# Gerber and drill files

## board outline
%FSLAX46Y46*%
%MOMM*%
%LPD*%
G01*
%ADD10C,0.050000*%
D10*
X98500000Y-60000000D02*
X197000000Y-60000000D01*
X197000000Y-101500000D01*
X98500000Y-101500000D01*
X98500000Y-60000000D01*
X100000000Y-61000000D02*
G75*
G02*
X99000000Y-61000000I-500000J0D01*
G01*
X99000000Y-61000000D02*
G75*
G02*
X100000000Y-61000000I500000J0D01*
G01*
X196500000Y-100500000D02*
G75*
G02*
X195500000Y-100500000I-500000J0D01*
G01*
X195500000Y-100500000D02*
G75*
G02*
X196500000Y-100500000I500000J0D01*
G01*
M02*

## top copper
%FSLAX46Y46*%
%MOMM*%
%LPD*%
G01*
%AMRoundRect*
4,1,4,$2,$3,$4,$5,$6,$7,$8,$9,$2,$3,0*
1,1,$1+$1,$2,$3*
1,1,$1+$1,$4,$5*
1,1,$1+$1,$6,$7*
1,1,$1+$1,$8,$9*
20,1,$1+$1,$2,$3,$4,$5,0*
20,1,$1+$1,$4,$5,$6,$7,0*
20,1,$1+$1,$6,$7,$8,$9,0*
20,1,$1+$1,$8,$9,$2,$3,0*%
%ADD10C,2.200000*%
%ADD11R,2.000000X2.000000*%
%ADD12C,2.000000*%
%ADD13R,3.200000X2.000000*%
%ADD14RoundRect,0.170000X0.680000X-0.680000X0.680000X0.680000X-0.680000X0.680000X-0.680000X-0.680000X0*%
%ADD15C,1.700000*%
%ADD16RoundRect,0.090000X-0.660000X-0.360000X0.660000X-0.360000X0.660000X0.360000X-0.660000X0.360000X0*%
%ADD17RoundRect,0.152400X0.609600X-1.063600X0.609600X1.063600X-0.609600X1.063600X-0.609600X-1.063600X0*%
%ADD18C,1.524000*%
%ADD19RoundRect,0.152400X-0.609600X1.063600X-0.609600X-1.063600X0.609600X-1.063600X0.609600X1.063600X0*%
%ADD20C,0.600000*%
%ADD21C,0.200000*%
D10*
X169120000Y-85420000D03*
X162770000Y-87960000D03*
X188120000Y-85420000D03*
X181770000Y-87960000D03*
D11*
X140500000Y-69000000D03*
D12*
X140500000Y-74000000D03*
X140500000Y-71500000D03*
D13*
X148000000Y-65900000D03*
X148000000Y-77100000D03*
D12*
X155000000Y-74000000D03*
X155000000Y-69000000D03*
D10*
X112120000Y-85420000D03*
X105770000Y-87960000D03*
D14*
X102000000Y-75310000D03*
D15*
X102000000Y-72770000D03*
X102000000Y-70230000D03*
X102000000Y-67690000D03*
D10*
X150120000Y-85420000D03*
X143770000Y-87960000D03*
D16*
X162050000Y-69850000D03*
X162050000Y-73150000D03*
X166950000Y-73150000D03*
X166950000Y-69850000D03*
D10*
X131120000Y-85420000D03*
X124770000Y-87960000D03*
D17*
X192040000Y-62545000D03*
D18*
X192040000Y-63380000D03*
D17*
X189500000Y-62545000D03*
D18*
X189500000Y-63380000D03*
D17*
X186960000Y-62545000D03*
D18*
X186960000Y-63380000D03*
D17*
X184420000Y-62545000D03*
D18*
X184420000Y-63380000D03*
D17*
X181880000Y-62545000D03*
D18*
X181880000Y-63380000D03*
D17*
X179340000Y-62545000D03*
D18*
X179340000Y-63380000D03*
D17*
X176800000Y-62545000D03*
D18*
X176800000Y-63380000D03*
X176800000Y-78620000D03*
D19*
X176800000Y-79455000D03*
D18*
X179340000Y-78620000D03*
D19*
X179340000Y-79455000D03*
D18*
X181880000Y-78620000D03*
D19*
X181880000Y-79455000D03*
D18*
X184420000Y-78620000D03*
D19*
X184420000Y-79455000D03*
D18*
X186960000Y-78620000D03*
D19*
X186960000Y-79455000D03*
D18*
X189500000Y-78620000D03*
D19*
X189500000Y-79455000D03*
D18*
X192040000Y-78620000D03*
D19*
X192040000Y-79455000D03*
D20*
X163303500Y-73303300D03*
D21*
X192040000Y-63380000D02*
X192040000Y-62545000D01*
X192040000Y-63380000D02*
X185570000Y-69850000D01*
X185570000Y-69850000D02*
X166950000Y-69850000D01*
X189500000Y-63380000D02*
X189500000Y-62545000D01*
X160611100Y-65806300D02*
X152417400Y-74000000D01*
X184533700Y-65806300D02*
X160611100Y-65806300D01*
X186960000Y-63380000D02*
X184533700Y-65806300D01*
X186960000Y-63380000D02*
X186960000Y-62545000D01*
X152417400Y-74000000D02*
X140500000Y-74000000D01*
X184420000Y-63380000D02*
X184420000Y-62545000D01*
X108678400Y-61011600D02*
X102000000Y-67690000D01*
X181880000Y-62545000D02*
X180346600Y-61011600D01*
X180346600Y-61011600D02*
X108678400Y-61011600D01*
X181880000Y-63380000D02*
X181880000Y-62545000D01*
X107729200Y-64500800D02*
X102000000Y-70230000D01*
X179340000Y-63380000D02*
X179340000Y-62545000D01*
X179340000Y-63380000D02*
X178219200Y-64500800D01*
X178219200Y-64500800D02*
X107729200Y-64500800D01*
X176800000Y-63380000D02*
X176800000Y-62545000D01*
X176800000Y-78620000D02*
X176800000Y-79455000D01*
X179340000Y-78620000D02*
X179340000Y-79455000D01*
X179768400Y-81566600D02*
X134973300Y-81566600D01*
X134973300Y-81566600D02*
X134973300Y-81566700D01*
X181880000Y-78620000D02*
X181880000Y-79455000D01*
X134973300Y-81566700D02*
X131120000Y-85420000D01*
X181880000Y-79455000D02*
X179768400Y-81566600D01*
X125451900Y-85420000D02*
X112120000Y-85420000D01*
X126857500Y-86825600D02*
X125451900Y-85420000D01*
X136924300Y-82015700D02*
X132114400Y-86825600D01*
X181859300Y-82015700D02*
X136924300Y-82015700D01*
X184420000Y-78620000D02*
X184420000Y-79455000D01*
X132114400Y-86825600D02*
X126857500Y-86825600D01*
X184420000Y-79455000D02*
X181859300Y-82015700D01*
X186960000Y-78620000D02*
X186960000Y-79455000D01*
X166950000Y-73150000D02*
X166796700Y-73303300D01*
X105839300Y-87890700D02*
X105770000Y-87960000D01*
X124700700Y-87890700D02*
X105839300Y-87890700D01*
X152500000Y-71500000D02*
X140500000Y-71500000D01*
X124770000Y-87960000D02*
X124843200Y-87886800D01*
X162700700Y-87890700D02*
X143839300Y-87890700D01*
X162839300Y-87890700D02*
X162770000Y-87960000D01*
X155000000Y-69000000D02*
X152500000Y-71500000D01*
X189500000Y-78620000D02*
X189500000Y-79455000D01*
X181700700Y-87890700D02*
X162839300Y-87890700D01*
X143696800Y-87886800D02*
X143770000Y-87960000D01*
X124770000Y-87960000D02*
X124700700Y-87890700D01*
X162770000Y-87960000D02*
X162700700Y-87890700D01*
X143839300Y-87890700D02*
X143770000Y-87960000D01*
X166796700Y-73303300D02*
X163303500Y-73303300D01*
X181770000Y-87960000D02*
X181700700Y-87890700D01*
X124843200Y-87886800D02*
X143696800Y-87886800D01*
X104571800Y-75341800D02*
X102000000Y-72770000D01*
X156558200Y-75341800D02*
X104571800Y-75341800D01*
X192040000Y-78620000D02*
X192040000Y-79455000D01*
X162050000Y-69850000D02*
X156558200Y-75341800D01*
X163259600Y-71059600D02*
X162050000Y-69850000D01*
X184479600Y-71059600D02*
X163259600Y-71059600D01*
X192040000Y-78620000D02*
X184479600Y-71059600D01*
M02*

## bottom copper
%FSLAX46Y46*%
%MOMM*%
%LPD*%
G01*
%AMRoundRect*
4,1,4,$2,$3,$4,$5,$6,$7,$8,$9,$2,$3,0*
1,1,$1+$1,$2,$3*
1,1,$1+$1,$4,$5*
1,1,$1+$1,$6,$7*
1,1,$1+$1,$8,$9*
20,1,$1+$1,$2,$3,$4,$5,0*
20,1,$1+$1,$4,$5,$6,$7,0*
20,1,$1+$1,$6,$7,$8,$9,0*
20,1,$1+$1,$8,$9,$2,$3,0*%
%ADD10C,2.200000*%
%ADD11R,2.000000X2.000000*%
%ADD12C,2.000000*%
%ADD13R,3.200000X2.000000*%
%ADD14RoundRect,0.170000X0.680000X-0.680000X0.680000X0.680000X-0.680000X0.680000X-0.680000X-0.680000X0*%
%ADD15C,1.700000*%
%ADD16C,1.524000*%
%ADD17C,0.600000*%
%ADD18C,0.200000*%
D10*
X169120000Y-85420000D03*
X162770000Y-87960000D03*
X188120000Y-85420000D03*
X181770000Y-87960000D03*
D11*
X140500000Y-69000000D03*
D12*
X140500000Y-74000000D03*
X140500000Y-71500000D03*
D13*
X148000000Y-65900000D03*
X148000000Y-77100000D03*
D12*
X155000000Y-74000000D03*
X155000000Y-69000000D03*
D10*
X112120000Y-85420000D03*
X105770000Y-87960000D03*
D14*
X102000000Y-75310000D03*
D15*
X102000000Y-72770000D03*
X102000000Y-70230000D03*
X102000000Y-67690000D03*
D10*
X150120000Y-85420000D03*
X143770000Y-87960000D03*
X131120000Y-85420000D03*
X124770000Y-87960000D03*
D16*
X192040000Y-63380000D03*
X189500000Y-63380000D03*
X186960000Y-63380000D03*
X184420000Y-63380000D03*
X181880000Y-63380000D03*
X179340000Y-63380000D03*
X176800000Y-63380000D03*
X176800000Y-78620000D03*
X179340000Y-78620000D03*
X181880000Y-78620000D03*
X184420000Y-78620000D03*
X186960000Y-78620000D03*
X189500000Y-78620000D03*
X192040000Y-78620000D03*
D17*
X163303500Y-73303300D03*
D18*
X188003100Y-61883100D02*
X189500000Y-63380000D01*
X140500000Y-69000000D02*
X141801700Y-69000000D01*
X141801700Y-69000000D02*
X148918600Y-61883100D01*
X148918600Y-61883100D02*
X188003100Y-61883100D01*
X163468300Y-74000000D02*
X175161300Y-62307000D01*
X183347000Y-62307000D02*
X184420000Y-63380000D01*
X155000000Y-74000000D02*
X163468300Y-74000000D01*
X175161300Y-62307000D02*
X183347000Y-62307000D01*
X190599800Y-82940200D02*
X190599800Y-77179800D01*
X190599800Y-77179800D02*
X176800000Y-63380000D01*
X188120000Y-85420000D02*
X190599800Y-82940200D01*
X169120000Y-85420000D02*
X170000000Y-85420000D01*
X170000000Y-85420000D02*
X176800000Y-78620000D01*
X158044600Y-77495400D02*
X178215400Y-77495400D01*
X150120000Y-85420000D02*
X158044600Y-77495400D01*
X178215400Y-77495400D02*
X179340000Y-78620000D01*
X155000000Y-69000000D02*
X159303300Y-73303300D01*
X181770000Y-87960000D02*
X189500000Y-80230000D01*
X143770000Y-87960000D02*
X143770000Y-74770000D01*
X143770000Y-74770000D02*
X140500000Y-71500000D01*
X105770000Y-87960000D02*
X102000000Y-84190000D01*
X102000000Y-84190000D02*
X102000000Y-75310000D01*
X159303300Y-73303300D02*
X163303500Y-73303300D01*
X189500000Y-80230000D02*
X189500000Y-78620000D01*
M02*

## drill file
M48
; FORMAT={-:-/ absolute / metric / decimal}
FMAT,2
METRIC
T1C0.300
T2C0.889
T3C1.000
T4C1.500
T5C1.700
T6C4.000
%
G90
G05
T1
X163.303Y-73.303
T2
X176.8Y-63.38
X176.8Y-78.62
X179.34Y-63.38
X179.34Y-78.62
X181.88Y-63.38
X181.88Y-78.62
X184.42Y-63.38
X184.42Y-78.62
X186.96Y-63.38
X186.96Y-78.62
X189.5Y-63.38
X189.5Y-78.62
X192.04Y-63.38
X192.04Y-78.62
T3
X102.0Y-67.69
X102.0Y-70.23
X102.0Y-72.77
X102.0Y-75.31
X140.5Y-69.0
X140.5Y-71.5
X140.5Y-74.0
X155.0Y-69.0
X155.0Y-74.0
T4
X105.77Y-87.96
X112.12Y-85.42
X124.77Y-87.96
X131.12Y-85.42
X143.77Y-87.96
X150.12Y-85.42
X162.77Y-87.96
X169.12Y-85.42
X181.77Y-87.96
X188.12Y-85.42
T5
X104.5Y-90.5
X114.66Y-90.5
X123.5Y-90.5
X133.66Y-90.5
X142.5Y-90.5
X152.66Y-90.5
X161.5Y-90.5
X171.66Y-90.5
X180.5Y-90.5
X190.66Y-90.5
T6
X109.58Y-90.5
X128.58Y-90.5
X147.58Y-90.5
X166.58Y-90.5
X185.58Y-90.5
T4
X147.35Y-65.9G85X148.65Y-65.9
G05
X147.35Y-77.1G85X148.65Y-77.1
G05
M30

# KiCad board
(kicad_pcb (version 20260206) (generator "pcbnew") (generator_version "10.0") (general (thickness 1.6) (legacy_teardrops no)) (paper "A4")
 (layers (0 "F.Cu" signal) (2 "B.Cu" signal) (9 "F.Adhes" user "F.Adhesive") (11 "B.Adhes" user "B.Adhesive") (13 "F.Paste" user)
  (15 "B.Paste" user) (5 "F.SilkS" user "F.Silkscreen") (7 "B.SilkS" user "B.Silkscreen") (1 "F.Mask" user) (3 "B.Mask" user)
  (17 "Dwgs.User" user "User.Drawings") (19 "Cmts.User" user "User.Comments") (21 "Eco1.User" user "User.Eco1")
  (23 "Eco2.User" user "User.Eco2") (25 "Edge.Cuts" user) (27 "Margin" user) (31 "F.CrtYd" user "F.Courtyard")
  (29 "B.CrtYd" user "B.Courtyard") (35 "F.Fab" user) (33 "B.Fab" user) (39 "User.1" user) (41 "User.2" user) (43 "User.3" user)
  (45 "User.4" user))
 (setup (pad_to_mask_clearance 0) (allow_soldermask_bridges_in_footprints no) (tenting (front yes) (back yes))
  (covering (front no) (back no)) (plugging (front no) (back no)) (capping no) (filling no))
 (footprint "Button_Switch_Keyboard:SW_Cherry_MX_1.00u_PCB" (layer "F.Cu") (at 169.12 85.42)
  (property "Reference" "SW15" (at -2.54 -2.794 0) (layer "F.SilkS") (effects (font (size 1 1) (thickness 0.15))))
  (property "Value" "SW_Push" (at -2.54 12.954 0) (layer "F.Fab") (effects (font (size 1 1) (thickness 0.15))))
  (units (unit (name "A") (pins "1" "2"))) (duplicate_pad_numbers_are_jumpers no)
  (pad "" np_thru_hole circle (at -7.62 5.08) (size 1.7 1.7) (drill 1.7) (layers "*.Cu" "*.Mask"))
  (pad "" np_thru_hole circle (at -2.54 5.08) (size 4 4) (drill 4) (layers "*.Cu" "*.Mask"))
  (pad "" np_thru_hole circle (at 2.54 5.08) (size 1.7 1.7) (drill 1.7) (layers "*.Cu" "*.Mask"))
  (pad "1" thru_hole circle (at 0 0) (size 2.2 2.2) (drill 1.5) (layers "*.Cu" "*.Mask") (remove_unused_layers no)
   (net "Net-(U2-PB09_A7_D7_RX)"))
  (pad "2" thru_hole circle (at -6.35 2.54) (size 2.2 2.2) (drill 1.5) (layers "*.Cu" "*.Mask") (remove_unused_layers no)
   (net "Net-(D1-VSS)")))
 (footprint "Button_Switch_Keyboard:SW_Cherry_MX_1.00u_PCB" (layer "F.Cu") (at 188.12 85.42)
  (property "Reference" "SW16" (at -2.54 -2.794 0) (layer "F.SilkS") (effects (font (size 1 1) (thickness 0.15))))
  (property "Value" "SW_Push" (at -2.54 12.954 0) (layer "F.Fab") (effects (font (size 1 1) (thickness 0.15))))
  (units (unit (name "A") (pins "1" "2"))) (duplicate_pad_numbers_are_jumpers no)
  (pad "" np_thru_hole circle (at -7.62 5.08) (size 1.7 1.7) (drill 1.7) (layers "*.Cu" "*.Mask"))
  (pad "" np_thru_hole circle (at -2.54 5.08) (size 4 4) (drill 4) (layers "*.Cu" "*.Mask"))
  (pad "" np_thru_hole circle (at 2.54 5.08) (size 1.7 1.7) (drill 1.7) (layers "*.Cu" "*.Mask"))
  (pad "1" thru_hole circle (at 0 0) (size 2.2 2.2) (drill 1.5) (layers "*.Cu" "*.Mask") (remove_unused_layers no)
   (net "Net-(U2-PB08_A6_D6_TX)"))
  (pad "2" thru_hole circle (at -6.35 2.54) (size 2.2 2.2) (drill 1.5) (layers "*.Cu" "*.Mask") (remove_unused_layers no)
   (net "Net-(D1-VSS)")))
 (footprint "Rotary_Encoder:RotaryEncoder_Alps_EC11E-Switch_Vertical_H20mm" (layer "F.Cu") (at 140.5 69)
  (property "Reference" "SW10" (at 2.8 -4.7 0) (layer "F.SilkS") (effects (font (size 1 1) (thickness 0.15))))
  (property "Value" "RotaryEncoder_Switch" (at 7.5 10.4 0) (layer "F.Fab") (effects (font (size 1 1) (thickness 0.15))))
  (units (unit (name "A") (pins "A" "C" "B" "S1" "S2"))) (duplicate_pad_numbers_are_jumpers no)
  (pad "A" thru_hole rect (at 0 0) (size 2 2) (drill 1) (layers "*.Cu" "*.Mask") (remove_unused_layers no) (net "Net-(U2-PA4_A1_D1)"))
  (pad "B" thru_hole circle (at 0 5) (size 2 2) (drill 1) (layers "*.Cu" "*.Mask") (remove_unused_layers no) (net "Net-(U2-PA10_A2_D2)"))
  (pad "C" thru_hole circle (at 0 2.5) (size 2 2) (drill 1) (layers "*.Cu" "*.Mask") (remove_unused_layers no) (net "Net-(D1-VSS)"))
  (pad "MP" thru_hole rect (at 7.5 -3.1) (size 3.2 2) (drill oval 2.8 1.5) (layers "*.Cu" "*.Mask") (remove_unused_layers no))
  (pad "MP" thru_hole rect (at 7.5 8.1) (size 3.2 2) (drill oval 2.8 1.5) (layers "*.Cu" "*.Mask") (remove_unused_layers no))
  (pad "S1" thru_hole circle (at 14.5 5) (size 2 2) (drill 1) (layers "*.Cu" "*.Mask") (remove_unused_layers no) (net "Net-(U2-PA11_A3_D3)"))
  (pad "S2" thru_hole circle (at 14.5 0) (size 2 2) (drill 1) (layers "*.Cu" "*.Mask") (remove_unused_layers no) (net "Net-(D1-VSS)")))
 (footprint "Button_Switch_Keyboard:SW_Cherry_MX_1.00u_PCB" (layer "F.Cu") (at 112.12 85.42)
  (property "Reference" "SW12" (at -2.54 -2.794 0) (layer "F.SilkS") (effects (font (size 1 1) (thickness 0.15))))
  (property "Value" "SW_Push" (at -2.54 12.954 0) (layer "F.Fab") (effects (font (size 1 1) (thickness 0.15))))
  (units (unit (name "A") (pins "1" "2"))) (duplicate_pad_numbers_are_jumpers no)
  (pad "" np_thru_hole circle (at -7.62 5.08) (size 1.7 1.7) (drill 1.7) (layers "*.Cu" "*.Mask"))
  (pad "" np_thru_hole circle (at -2.54 5.08) (size 4 4) (drill 4) (layers "*.Cu" "*.Mask"))
  (pad "" np_thru_hole circle (at 2.54 5.08) (size 1.7 1.7) (drill 1.7) (layers "*.Cu" "*.Mask"))
  (pad "1" thru_hole circle (at 0 0) (size 2.2 2.2) (drill 1.5) (layers "*.Cu" "*.Mask") (remove_unused_layers no)
   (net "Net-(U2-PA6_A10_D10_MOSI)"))
  (pad "2" thru_hole circle (at -6.35 2.54) (size 2.2 2.2) (drill 1.5) (layers "*.Cu" "*.Mask") (remove_unused_layers no)
   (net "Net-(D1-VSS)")))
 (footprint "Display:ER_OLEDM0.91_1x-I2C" (layer "F.Cu") (at 102 75.31 90)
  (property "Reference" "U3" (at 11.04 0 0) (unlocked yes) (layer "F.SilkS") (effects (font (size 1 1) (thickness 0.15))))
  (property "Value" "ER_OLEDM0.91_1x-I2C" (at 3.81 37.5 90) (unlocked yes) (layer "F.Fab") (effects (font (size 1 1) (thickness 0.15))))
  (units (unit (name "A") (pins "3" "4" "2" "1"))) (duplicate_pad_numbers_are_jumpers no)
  (pad "1" thru_hole roundrect (at 0 0 90) (size 1.7 1.7) (drill 1) (layers "*.Cu" "*.Mask") (remove_unused_layers no)
   (roundrect_rratio 0.1) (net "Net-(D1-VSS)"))
  (pad "2" thru_hole circle (at 2.54 0 90) (size 1.7 1.7) (drill 1) (layers "*.Cu" "*.Mask") (remove_unused_layers no) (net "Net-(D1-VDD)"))
  (pad "3" thru_hole circle (at 5.08 0 90) (size 1.7 1.7) (drill 1) (layers "*.Cu" "*.Mask") (remove_unused_layers no)
   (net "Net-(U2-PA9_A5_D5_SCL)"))
  (pad "4" thru_hole circle (at 7.62 0 90) (size 1.7 1.7) (drill 1) (layers "*.Cu" "*.Mask") (remove_unused_layers no)
   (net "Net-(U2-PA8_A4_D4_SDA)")))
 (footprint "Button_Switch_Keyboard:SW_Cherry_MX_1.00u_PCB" (layer "F.Cu") (at 150.12 85.42)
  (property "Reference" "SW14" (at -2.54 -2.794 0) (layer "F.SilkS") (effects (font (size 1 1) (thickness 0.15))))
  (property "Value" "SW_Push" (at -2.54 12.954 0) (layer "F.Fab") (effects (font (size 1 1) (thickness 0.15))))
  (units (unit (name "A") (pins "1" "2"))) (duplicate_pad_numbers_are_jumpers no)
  (pad "" np_thru_hole circle (at -7.62 5.08) (size 1.7 1.7) (drill 1.7) (layers "*.Cu" "*.Mask"))
  (pad "" np_thru_hole circle (at -2.54 5.08) (size 4 4) (drill 4) (layers "*.Cu" "*.Mask"))
  (pad "" np_thru_hole circle (at 2.54 5.08) (size 1.7 1.7) (drill 1.7) (layers "*.Cu" "*.Mask"))
  (pad "1" thru_hole circle (at 0 0) (size 2.2 2.2) (drill 1.5) (layers "*.Cu" "*.Mask") (remove_unused_layers no)
   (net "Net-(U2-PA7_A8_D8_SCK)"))
  (pad "2" thru_hole circle (at -6.35 2.54) (size 2.2 2.2) (drill 1.5) (layers "*.Cu" "*.Mask") (remove_unused_layers no)
   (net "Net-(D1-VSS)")))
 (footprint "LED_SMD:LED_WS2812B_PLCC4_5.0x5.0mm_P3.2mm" (layer "F.Cu") (at 164.5 71.5)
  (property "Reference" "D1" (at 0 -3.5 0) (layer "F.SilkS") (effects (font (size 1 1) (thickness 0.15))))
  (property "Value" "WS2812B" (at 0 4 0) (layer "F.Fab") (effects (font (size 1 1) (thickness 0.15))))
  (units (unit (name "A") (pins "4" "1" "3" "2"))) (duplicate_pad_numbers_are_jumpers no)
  (pad "1" smd roundrect (at -2.45 -1.65) (size 1.5 0.9) (layers "F.Cu" "F.Mask" "F.Paste") (roundrect_rratio 0.1) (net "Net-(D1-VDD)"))
  (pad "2" smd roundrect (at -2.45 1.65) (size 1.5 0.9) (layers "F.Cu" "F.Mask" "F.Paste") (roundrect_rratio 0.1)
   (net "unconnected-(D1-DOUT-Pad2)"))
  (pad "3" smd roundrect (at 2.45 1.65) (size 1.5 0.9) (layers "F.Cu" "F.Mask" "F.Paste") (roundrect_rratio 0.1) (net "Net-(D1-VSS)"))
  (pad "4" smd roundrect (at 2.45 -1.65) (size 1.5 0.9) (layers "F.Cu" "F.Mask" "F.Paste") (roundrect_rratio 0.1) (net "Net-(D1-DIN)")))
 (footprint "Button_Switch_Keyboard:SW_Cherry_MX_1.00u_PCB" (layer "F.Cu") (at 131.12 85.42)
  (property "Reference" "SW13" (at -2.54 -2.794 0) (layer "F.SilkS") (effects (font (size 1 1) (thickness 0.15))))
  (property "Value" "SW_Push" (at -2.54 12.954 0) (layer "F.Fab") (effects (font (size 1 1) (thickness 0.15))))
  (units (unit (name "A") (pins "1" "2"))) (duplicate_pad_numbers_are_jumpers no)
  (pad "" np_thru_hole circle (at -7.62 5.08) (size 1.7 1.7) (drill 1.7) (layers "*.Cu" "*.Mask"))
  (pad "" np_thru_hole circle (at -2.54 5.08) (size 4 4) (drill 4) (layers "*.Cu" "*.Mask"))
  (pad "" np_thru_hole circle (at 2.54 5.08) (size 1.7 1.7) (drill 1.7) (layers "*.Cu" "*.Mask"))
  (pad "1" thru_hole circle (at 0 0) (size 2.2 2.2) (drill 1.5) (layers "*.Cu" "*.Mask") (remove_unused_layers no)
   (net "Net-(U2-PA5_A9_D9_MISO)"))
  (pad "2" thru_hole circle (at -6.35 2.54) (size 2.2 2.2) (drill 1.5) (layers "*.Cu" "*.Mask") (remove_unused_layers no)
   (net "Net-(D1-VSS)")))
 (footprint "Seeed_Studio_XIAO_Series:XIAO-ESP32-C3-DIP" (layer "F.Cu") (at 184.42 71)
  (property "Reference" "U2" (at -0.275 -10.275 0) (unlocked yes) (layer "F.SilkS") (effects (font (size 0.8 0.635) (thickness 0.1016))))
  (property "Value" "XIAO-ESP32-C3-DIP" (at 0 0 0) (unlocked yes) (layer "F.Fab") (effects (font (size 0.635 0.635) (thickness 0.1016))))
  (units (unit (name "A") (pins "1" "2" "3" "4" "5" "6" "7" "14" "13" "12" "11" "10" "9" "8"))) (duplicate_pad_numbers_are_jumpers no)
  (pad "1" smd roundrect (at 7.62 -8.455 90) (size 2.432 1.524) (layers "F.Cu" "F.Mask") (roundrect_rratio 0.1) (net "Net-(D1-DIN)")
   (thermal_bridge_angle 45))
  (pad "1" thru_hole circle (at 7.62 -7.62 90) (size 1.524 1.524) (drill 0.889) (layers "*.Cu" "*.Mask") (remove_unused_layers no)
   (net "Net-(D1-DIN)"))
  (pad "2" smd roundrect (at 5.08 -8.455 90) (size 2.432 1.524) (layers "F.Cu" "F.Mask") (roundrect_rratio 0.1) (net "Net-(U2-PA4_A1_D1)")
   (thermal_bridge_angle 45))
  (pad "2" thru_hole circle (at 5.08 -7.62 90) (size 1.524 1.524) (drill 0.889) (layers "*.Cu" "*.Mask") (remove_unused_layers no)
   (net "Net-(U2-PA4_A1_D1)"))
  (pad "3" smd roundrect (at 2.54 -8.455 90) (size 2.432 1.524) (layers "F.Cu" "F.Mask") (roundrect_rratio 0.1) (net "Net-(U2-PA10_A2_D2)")
   (thermal_bridge_angle 45))
  (pad "3" thru_hole circle (at 2.54 -7.62 90) (size 1.524 1.524) (drill 0.889) (layers "*.Cu" "*.Mask") (remove_unused_layers no)
   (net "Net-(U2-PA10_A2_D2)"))
  (pad "4" smd roundrect (at 0 -8.455 90) (size 2.432 1.524) (layers "F.Cu" "F.Mask") (roundrect_rratio 0.1) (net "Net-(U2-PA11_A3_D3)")
   (thermal_bridge_angle 45))
  (pad "4" thru_hole circle (at 0 -7.62 90) (size 1.524 1.524) (drill 0.889) (layers "*.Cu" "*.Mask") (remove_unused_layers no)
   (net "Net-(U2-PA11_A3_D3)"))
  (pad "5" smd roundrect (at -2.54 -8.455 90) (size 2.432 1.524) (layers "F.Cu" "F.Mask") (roundrect_rratio 0.1)
   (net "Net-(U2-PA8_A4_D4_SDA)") (thermal_bridge_angle 45))
  (pad "5" thru_hole circle (at -2.54 -7.62 90) (size 1.524 1.524) (drill 0.889) (layers "*.Cu" "*.Mask") (remove_unused_layers no)
   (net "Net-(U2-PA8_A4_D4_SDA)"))
  (pad "6" smd roundrect (at -5.08 -8.455 90) (size 2.432 1.524) (layers "F.Cu" "F.Mask") (roundrect_rratio 0.1)
   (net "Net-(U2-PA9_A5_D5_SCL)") (thermal_bridge_angle 45))
  (pad "6" thru_hole circle (at -5.08 -7.62 90) (size 1.524 1.524) (drill 0.889) (layers "*.Cu" "*.Mask") (remove_unused_layers no)
   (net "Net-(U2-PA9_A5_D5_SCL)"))
  (pad "7" smd roundrect (at -7.62 -8.455 90) (size 2.432 1.524) (layers "F.Cu" "F.Mask") (roundrect_rratio 0.1)
   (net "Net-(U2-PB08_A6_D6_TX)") (thermal_bridge_angle 45))
  (pad "7" thru_hole circle (at -7.62 -7.62 90) (size 1.524 1.524) (drill 0.889) (layers "*.Cu" "*.Mask") (remove_unused_layers no)
   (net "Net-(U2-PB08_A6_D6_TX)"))
  (pad "8" thru_hole circle (at -7.62 7.62 270) (size 1.524 1.524) (drill 0.889) (layers "*.Cu" "*.Mask") (remove_unused_layers no)
   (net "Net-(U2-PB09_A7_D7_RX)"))
  (pad "8" smd roundrect (at -7.62 8.455 270) (size 2.432 1.524) (layers "F.Cu" "F.Mask") (roundrect_rratio 0.1)
   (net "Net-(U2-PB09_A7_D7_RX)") (thermal_bridge_angle 45))
  (pad "9" thru_hole circle (at -5.08 7.62 270) (size 1.524 1.524) (drill 0.889) (layers "*.Cu" "*.Mask") (remove_unused_layers no)
   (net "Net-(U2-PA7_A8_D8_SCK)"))
  (pad "9" smd roundrect (at -5.08 8.455 270) (size 2.432 1.524) (layers "F.Cu" "F.Mask") (roundrect_rratio 0.1)
   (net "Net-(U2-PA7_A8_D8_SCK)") (thermal_bridge_angle 45))
  (pad "10" thru_hole circle (at -2.54 7.62 270) (size 1.524 1.524) (drill 0.889) (layers "*.Cu" "*.Mask") (remove_unused_layers no)
   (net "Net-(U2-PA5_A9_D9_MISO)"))
  (pad "10" smd roundrect (at -2.54 8.455 270) (size 2.432 1.524) (layers "F.Cu" "F.Mask") (roundrect_rratio 0.1)
   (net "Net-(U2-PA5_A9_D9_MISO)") (thermal_bridge_angle 45))
  (pad "11" thru_hole circle (at 0 7.62 270) (size 1.524 1.524) (drill 0.889) (layers "*.Cu" "*.Mask") (remove_unused_layers no)
   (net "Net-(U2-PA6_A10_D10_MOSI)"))
  (pad "11" smd roundrect (at 0 8.455 270) (size 2.432 1.524) (layers "F.Cu" "F.Mask") (roundrect_rratio 0.1)
   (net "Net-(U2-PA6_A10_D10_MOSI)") (thermal_bridge_angle 45))
  (pad "12" thru_hole circle (at 2.54 7.62 270) (size 1.524 1.524) (drill 0.889) (layers "*.Cu" "*.Mask") (remove_unused_layers no)
   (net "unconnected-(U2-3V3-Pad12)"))
  (pad "12" smd roundrect (at 2.54 8.455 270) (size 2.432 1.524) (layers "F.Cu" "F.Mask") (roundrect_rratio 0.1)
   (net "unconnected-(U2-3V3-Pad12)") (thermal_bridge_angle 45))
  (pad "13" thru_hole circle (at 5.08 7.62 270) (size 1.524 1.524) (drill 0.889) (layers "*.Cu" "*.Mask") (remove_unused_layers no)
   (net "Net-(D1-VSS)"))
  (pad "13" smd roundrect (at 5.08 8.455 270) (size 2.432 1.524) (layers "F.Cu" "F.Mask") (roundrect_rratio 0.1) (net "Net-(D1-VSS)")
   (thermal_bridge_angle 45))
  (pad "14" thru_hole circle (at 7.62 7.62 270) (size 1.524 1.524) (drill 0.889) (layers "*.Cu" "*.Mask") (remove_unused_layers no)
   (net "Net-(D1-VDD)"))
  (pad "14" smd roundrect (at 7.62 8.455 270) (size 2.432 1.524) (layers "F.Cu" "F.Mask") (roundrect_rratio 0.1) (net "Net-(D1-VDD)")
   (thermal_bridge_angle 45)))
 (gr_rect (start 98.5 60) (end 197 101.5) (stroke (width 0.05) (type default)) (fill no) (layer "Edge.Cuts"))
 (gr_circle (center 99.5 61) (end 99.5 60.5) (stroke (width 0.05) (type default)) (fill no) (layer "Edge.Cuts"))
 (gr_circle (center 196 100.5) (end 196 101) (stroke (width 0.05) (type default)) (fill no) (layer "Edge.Cuts"))
 (segment (start 192.04 63.38) (end 192.04 62.545) (width 0.2) (layer "F.Cu") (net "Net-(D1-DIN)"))
 (segment (start 192.04 63.38) (end 185.57 69.85) (width 0.2) (layer "F.Cu") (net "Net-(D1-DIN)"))
 (segment (start 185.57 69.85) (end 166.95 69.85) (width 0.2) (layer "F.Cu") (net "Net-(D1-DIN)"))
 (segment (start 189.5 63.38) (end 189.5 62.545) (width 0.2) (layer "F.Cu") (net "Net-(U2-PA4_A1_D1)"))
 (segment (start 188.0031 61.8831) (end 189.5 63.38) (width 0.2) (layer "B.Cu") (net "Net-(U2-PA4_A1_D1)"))
 (segment (start 140.5 69) (end 141.8017 69) (width 0.2) (layer "B.Cu") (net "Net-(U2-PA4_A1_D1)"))
 (segment (start 141.8017 69) (end 148.9186 61.8831) (width 0.2) (layer "B.Cu") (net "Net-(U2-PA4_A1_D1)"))
 (segment (start 148.9186 61.8831) (end 188.0031 61.8831) (width 0.2) (layer "B.Cu") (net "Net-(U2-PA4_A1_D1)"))
 (segment (start 160.6111 65.8063) (end 152.4174 74) (width 0.2) (layer "F.Cu") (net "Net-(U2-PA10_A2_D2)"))
 (segment (start 184.5337 65.8063) (end 160.6111 65.8063) (width 0.2) (layer "F.Cu") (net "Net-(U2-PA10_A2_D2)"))
 (segment (start 186.96 63.38) (end 184.5337 65.8063) (width 0.2) (layer "F.Cu") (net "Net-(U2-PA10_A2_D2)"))
 (segment (start 186.96 63.38) (end 186.96 62.545) (width 0.2) (layer "F.Cu") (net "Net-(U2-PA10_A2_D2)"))
 (segment (start 152.4174 74) (end 140.5 74) (width 0.2) (layer "F.Cu") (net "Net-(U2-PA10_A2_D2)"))
 (segment (start 184.42 63.38) (end 184.42 62.545) (width 0.2) (layer "F.Cu") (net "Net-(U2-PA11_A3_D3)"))
 (segment (start 163.4683 74) (end 175.1613 62.307) (width 0.2) (layer "B.Cu") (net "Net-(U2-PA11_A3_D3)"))
 (segment (start 183.347 62.307) (end 184.42 63.38) (width 0.2) (layer "B.Cu") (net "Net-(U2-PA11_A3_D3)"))
 (segment (start 155 74) (end 163.4683 74) (width 0.2) (layer "B.Cu") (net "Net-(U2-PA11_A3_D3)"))
 (segment (start 175.1613 62.307) (end 183.347 62.307) (width 0.2) (layer "B.Cu") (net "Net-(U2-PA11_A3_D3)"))
 (segment (start 108.6784 61.0116) (end 102 67.69) (width 0.2) (layer "F.Cu") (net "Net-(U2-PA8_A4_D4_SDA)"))
 (segment (start 181.88 62.545) (end 180.3466 61.0116) (width 0.2) (layer "F.Cu") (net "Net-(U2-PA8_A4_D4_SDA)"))
 (segment (start 180.3466 61.0116) (end 108.6784 61.0116) (width 0.2) (layer "F.Cu") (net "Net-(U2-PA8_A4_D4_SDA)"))
 (segment (start 181.88 63.38) (end 181.88 62.545) (width 0.2) (layer "F.Cu") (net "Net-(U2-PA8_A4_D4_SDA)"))
 (segment (start 107.7292 64.5008) (end 102 70.23) (width 0.2) (layer "F.Cu") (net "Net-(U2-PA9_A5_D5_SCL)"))
 (segment (start 179.34 63.38) (end 179.34 62.545) (width 0.2) (layer "F.Cu") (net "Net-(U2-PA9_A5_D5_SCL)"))
 (segment (start 179.34 63.38) (end 178.2192 64.5008) (width 0.2) (layer "F.Cu") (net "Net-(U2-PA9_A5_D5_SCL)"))
 (segment (start 178.2192 64.5008) (end 107.7292 64.5008) (width 0.2) (layer "F.Cu") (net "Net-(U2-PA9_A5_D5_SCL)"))
 (segment (start 176.8 63.38) (end 176.8 62.545) (width 0.2) (layer "F.Cu") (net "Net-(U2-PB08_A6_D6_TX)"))
 (segment (start 190.5998 82.9402) (end 190.5998 77.1798) (width 0.2) (layer "B.Cu") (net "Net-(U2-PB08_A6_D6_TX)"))
 (segment (start 190.5998 77.1798) (end 176.8 63.38) (width 0.2) (layer "B.Cu") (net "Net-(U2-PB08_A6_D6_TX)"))
 (segment (start 188.12 85.42) (end 190.5998 82.9402) (width 0.2) (layer "B.Cu") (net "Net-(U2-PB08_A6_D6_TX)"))
 (segment (start 176.8 78.62) (end 176.8 79.455) (width 0.2) (layer "F.Cu") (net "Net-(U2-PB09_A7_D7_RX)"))
 (segment (start 169.12 85.42) (end 170 85.42) (width 0.2) (layer "B.Cu") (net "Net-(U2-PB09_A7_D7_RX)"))
 (segment (start 170 85.42) (end 176.8 78.62) (width 0.2) (layer "B.Cu") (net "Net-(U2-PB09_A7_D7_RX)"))
 (segment (start 179.34 78.62) (end 179.34 79.455) (width 0.2) (layer "F.Cu") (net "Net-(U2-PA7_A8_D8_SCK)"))
 (segment (start 158.0446 77.4954) (end 178.2154 77.4954) (width 0.2) (layer "B.Cu") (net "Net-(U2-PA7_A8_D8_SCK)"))
 (segment (start 150.12 85.42) (end 158.0446 77.4954) (width 0.2) (layer "B.Cu") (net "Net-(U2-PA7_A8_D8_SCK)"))
 (segment (start 178.2154 77.4954) (end 179.34 78.62) (width 0.2) (layer "B.Cu") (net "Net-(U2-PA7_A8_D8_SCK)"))
 (segment (start 179.7684 81.5666) (end 134.9733 81.5666) (width 0.2) (layer "F.Cu") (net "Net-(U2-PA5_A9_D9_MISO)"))
 (segment (start 134.9733 81.5666) (end 134.9733 81.5667) (width 0.2) (layer "F.Cu") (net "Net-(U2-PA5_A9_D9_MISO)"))
 (segment (start 181.88 78.62) (end 181.88 79.455) (width 0.2) (layer "F.Cu") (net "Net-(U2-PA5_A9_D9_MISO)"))
 (segment (start 134.9733 81.5667) (end 131.12 85.42) (width 0.2) (layer "F.Cu") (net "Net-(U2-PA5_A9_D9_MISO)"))
 (segment (start 181.88 79.455) (end 179.7684 81.5666) (width 0.2) (layer "F.Cu") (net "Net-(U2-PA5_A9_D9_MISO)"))
 (segment (start 125.4519 85.42) (end 112.12 85.42) (width 0.2) (layer "F.Cu") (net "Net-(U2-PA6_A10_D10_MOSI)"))
 (segment (start 126.8575 86.8256) (end 125.4519 85.42) (width 0.2) (layer "F.Cu") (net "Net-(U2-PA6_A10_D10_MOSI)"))
 (segment (start 136.9243 82.0157) (end 132.1144 86.8256) (width 0.2) (layer "F.Cu") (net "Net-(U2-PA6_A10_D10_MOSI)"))
 (segment (start 181.8593 82.0157) (end 136.9243 82.0157) (width 0.2) (layer "F.Cu") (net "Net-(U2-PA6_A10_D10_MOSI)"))
 (segment (start 184.42 78.62) (end 184.42 79.455) (width 0.2) (layer "F.Cu") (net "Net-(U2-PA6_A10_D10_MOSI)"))
 (segment (start 132.1144 86.8256) (end 126.8575 86.8256) (width 0.2) (layer "F.Cu") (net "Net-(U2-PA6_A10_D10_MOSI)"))
 (segment (start 184.42 79.455) (end 181.8593 82.0157) (width 0.2) (layer "F.Cu") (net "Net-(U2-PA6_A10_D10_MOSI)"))
 (segment (start 186.96 78.62) (end 186.96 79.455) (width 0.2) (layer "F.Cu") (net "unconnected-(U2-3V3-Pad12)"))
 (segment (start 166.95 73.15) (end 166.7967 73.3033) (width 0.2) (layer "F.Cu") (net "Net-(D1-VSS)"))
 (segment (start 105.8393 87.8907) (end 105.77 87.96) (width 0.2) (layer "F.Cu") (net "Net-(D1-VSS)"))
 (segment (start 124.7007 87.8907) (end 105.8393 87.8907) (width 0.2) (layer "F.Cu") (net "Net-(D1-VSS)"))
 (segment (start 152.5 71.5) (end 140.5 71.5) (width 0.2) (layer "F.Cu") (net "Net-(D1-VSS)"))
 (segment (start 124.77 87.96) (end 124.8432 87.8868) (width 0.2) (layer "F.Cu") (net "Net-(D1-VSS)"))
 (segment (start 162.7007 87.8907) (end 143.8393 87.8907) (width 0.2) (layer "F.Cu") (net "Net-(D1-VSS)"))
 (segment (start 162.8393 87.8907) (end 162.77 87.96) (width 0.2) (layer "F.Cu") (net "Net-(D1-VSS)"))
 (segment (start 155 69) (end 152.5 71.5) (width 0.2) (layer "F.Cu") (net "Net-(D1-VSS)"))
 (segment (start 189.5 78.62) (end 189.5 79.455) (width 0.2) (layer "F.Cu") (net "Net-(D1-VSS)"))
 (segment (start 181.7007 87.8907) (end 162.8393 87.8907) (width 0.2) (layer "F.Cu") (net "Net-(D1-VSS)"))
 (segment (start 143.6968 87.8868) (end 143.77 87.96) (width 0.2) (layer "F.Cu") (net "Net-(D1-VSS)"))
 (segment (start 124.77 87.96) (end 124.7007 87.8907) (width 0.2) (layer "F.Cu") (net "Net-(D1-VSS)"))
 (segment (start 162.77 87.96) (end 162.7007 87.8907) (width 0.2) (layer "F.Cu") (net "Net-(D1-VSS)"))
 (segment (start 143.8393 87.8907) (end 143.77 87.96) (width 0.2) (layer "F.Cu") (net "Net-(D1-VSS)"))
 (segment (start 166.7967 73.3033) (end 163.3035 73.3033) (width 0.2) (layer "F.Cu") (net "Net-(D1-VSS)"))
 (segment (start 181.77 87.96) (end 181.7007 87.8907) (width 0.2) (layer "F.Cu") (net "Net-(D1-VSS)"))
 (segment (start 124.8432 87.8868) (end 143.6968 87.8868) (width 0.2) (layer "F.Cu") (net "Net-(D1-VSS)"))
 (via (at 163.3035 73.3033) (size 0.6) (drill 0.3) (layers "F.Cu" "B.Cu") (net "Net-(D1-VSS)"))
 (segment (start 155 69) (end 159.3033 73.3033) (width 0.2) (layer "B.Cu") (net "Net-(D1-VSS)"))
 (segment (start 181.77 87.96) (end 189.5 80.23) (width 0.2) (layer "B.Cu") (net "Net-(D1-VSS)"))
 (segment (start 143.77 87.96) (end 143.77 74.77) (width 0.2) (layer "B.Cu") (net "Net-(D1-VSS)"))
 (segment (start 143.77 74.77) (end 140.5 71.5) (width 0.2) (layer "B.Cu") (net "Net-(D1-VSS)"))
 (segment (start 105.77 87.96) (end 102 84.19) (width 0.2) (layer "B.Cu") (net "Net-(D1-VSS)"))
 (segment (start 102 84.19) (end 102 75.31) (width 0.2) (layer "B.Cu") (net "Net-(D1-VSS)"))
 (segment (start 159.3033 73.3033) (end 163.3035 73.3033) (width 0.2) (layer "B.Cu") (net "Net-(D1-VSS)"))
 (segment (start 189.5 80.23) (end 189.5 78.62) (width 0.2) (layer "B.Cu") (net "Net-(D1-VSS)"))
 (segment (start 104.5718 75.3418) (end 102 72.77) (width 0.2) (layer "F.Cu") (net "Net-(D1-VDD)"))
 (segment (start 156.5582 75.3418) (end 104.5718 75.3418) (width 0.2) (layer "F.Cu") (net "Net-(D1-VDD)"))
 (segment (start 192.04 78.62) (end 192.04 79.455) (width 0.2) (layer "F.Cu") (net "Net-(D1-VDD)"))
 (segment (start 162.05 69.85) (end 156.5582 75.3418) (width 0.2) (layer "F.Cu") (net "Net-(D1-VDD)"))
 (segment (start 163.2596 71.0596) (end 162.05 69.85) (width 0.2) (layer "F.Cu") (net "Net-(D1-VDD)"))
 (segment (start 184.4796 71.0596) (end 163.2596 71.0596) (width 0.2) (layer "F.Cu") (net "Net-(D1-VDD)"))
 (segment (start 192.04 78.62) (end 184.4796 71.0596) (width 0.2) (layer "F.Cu") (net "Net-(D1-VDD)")))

